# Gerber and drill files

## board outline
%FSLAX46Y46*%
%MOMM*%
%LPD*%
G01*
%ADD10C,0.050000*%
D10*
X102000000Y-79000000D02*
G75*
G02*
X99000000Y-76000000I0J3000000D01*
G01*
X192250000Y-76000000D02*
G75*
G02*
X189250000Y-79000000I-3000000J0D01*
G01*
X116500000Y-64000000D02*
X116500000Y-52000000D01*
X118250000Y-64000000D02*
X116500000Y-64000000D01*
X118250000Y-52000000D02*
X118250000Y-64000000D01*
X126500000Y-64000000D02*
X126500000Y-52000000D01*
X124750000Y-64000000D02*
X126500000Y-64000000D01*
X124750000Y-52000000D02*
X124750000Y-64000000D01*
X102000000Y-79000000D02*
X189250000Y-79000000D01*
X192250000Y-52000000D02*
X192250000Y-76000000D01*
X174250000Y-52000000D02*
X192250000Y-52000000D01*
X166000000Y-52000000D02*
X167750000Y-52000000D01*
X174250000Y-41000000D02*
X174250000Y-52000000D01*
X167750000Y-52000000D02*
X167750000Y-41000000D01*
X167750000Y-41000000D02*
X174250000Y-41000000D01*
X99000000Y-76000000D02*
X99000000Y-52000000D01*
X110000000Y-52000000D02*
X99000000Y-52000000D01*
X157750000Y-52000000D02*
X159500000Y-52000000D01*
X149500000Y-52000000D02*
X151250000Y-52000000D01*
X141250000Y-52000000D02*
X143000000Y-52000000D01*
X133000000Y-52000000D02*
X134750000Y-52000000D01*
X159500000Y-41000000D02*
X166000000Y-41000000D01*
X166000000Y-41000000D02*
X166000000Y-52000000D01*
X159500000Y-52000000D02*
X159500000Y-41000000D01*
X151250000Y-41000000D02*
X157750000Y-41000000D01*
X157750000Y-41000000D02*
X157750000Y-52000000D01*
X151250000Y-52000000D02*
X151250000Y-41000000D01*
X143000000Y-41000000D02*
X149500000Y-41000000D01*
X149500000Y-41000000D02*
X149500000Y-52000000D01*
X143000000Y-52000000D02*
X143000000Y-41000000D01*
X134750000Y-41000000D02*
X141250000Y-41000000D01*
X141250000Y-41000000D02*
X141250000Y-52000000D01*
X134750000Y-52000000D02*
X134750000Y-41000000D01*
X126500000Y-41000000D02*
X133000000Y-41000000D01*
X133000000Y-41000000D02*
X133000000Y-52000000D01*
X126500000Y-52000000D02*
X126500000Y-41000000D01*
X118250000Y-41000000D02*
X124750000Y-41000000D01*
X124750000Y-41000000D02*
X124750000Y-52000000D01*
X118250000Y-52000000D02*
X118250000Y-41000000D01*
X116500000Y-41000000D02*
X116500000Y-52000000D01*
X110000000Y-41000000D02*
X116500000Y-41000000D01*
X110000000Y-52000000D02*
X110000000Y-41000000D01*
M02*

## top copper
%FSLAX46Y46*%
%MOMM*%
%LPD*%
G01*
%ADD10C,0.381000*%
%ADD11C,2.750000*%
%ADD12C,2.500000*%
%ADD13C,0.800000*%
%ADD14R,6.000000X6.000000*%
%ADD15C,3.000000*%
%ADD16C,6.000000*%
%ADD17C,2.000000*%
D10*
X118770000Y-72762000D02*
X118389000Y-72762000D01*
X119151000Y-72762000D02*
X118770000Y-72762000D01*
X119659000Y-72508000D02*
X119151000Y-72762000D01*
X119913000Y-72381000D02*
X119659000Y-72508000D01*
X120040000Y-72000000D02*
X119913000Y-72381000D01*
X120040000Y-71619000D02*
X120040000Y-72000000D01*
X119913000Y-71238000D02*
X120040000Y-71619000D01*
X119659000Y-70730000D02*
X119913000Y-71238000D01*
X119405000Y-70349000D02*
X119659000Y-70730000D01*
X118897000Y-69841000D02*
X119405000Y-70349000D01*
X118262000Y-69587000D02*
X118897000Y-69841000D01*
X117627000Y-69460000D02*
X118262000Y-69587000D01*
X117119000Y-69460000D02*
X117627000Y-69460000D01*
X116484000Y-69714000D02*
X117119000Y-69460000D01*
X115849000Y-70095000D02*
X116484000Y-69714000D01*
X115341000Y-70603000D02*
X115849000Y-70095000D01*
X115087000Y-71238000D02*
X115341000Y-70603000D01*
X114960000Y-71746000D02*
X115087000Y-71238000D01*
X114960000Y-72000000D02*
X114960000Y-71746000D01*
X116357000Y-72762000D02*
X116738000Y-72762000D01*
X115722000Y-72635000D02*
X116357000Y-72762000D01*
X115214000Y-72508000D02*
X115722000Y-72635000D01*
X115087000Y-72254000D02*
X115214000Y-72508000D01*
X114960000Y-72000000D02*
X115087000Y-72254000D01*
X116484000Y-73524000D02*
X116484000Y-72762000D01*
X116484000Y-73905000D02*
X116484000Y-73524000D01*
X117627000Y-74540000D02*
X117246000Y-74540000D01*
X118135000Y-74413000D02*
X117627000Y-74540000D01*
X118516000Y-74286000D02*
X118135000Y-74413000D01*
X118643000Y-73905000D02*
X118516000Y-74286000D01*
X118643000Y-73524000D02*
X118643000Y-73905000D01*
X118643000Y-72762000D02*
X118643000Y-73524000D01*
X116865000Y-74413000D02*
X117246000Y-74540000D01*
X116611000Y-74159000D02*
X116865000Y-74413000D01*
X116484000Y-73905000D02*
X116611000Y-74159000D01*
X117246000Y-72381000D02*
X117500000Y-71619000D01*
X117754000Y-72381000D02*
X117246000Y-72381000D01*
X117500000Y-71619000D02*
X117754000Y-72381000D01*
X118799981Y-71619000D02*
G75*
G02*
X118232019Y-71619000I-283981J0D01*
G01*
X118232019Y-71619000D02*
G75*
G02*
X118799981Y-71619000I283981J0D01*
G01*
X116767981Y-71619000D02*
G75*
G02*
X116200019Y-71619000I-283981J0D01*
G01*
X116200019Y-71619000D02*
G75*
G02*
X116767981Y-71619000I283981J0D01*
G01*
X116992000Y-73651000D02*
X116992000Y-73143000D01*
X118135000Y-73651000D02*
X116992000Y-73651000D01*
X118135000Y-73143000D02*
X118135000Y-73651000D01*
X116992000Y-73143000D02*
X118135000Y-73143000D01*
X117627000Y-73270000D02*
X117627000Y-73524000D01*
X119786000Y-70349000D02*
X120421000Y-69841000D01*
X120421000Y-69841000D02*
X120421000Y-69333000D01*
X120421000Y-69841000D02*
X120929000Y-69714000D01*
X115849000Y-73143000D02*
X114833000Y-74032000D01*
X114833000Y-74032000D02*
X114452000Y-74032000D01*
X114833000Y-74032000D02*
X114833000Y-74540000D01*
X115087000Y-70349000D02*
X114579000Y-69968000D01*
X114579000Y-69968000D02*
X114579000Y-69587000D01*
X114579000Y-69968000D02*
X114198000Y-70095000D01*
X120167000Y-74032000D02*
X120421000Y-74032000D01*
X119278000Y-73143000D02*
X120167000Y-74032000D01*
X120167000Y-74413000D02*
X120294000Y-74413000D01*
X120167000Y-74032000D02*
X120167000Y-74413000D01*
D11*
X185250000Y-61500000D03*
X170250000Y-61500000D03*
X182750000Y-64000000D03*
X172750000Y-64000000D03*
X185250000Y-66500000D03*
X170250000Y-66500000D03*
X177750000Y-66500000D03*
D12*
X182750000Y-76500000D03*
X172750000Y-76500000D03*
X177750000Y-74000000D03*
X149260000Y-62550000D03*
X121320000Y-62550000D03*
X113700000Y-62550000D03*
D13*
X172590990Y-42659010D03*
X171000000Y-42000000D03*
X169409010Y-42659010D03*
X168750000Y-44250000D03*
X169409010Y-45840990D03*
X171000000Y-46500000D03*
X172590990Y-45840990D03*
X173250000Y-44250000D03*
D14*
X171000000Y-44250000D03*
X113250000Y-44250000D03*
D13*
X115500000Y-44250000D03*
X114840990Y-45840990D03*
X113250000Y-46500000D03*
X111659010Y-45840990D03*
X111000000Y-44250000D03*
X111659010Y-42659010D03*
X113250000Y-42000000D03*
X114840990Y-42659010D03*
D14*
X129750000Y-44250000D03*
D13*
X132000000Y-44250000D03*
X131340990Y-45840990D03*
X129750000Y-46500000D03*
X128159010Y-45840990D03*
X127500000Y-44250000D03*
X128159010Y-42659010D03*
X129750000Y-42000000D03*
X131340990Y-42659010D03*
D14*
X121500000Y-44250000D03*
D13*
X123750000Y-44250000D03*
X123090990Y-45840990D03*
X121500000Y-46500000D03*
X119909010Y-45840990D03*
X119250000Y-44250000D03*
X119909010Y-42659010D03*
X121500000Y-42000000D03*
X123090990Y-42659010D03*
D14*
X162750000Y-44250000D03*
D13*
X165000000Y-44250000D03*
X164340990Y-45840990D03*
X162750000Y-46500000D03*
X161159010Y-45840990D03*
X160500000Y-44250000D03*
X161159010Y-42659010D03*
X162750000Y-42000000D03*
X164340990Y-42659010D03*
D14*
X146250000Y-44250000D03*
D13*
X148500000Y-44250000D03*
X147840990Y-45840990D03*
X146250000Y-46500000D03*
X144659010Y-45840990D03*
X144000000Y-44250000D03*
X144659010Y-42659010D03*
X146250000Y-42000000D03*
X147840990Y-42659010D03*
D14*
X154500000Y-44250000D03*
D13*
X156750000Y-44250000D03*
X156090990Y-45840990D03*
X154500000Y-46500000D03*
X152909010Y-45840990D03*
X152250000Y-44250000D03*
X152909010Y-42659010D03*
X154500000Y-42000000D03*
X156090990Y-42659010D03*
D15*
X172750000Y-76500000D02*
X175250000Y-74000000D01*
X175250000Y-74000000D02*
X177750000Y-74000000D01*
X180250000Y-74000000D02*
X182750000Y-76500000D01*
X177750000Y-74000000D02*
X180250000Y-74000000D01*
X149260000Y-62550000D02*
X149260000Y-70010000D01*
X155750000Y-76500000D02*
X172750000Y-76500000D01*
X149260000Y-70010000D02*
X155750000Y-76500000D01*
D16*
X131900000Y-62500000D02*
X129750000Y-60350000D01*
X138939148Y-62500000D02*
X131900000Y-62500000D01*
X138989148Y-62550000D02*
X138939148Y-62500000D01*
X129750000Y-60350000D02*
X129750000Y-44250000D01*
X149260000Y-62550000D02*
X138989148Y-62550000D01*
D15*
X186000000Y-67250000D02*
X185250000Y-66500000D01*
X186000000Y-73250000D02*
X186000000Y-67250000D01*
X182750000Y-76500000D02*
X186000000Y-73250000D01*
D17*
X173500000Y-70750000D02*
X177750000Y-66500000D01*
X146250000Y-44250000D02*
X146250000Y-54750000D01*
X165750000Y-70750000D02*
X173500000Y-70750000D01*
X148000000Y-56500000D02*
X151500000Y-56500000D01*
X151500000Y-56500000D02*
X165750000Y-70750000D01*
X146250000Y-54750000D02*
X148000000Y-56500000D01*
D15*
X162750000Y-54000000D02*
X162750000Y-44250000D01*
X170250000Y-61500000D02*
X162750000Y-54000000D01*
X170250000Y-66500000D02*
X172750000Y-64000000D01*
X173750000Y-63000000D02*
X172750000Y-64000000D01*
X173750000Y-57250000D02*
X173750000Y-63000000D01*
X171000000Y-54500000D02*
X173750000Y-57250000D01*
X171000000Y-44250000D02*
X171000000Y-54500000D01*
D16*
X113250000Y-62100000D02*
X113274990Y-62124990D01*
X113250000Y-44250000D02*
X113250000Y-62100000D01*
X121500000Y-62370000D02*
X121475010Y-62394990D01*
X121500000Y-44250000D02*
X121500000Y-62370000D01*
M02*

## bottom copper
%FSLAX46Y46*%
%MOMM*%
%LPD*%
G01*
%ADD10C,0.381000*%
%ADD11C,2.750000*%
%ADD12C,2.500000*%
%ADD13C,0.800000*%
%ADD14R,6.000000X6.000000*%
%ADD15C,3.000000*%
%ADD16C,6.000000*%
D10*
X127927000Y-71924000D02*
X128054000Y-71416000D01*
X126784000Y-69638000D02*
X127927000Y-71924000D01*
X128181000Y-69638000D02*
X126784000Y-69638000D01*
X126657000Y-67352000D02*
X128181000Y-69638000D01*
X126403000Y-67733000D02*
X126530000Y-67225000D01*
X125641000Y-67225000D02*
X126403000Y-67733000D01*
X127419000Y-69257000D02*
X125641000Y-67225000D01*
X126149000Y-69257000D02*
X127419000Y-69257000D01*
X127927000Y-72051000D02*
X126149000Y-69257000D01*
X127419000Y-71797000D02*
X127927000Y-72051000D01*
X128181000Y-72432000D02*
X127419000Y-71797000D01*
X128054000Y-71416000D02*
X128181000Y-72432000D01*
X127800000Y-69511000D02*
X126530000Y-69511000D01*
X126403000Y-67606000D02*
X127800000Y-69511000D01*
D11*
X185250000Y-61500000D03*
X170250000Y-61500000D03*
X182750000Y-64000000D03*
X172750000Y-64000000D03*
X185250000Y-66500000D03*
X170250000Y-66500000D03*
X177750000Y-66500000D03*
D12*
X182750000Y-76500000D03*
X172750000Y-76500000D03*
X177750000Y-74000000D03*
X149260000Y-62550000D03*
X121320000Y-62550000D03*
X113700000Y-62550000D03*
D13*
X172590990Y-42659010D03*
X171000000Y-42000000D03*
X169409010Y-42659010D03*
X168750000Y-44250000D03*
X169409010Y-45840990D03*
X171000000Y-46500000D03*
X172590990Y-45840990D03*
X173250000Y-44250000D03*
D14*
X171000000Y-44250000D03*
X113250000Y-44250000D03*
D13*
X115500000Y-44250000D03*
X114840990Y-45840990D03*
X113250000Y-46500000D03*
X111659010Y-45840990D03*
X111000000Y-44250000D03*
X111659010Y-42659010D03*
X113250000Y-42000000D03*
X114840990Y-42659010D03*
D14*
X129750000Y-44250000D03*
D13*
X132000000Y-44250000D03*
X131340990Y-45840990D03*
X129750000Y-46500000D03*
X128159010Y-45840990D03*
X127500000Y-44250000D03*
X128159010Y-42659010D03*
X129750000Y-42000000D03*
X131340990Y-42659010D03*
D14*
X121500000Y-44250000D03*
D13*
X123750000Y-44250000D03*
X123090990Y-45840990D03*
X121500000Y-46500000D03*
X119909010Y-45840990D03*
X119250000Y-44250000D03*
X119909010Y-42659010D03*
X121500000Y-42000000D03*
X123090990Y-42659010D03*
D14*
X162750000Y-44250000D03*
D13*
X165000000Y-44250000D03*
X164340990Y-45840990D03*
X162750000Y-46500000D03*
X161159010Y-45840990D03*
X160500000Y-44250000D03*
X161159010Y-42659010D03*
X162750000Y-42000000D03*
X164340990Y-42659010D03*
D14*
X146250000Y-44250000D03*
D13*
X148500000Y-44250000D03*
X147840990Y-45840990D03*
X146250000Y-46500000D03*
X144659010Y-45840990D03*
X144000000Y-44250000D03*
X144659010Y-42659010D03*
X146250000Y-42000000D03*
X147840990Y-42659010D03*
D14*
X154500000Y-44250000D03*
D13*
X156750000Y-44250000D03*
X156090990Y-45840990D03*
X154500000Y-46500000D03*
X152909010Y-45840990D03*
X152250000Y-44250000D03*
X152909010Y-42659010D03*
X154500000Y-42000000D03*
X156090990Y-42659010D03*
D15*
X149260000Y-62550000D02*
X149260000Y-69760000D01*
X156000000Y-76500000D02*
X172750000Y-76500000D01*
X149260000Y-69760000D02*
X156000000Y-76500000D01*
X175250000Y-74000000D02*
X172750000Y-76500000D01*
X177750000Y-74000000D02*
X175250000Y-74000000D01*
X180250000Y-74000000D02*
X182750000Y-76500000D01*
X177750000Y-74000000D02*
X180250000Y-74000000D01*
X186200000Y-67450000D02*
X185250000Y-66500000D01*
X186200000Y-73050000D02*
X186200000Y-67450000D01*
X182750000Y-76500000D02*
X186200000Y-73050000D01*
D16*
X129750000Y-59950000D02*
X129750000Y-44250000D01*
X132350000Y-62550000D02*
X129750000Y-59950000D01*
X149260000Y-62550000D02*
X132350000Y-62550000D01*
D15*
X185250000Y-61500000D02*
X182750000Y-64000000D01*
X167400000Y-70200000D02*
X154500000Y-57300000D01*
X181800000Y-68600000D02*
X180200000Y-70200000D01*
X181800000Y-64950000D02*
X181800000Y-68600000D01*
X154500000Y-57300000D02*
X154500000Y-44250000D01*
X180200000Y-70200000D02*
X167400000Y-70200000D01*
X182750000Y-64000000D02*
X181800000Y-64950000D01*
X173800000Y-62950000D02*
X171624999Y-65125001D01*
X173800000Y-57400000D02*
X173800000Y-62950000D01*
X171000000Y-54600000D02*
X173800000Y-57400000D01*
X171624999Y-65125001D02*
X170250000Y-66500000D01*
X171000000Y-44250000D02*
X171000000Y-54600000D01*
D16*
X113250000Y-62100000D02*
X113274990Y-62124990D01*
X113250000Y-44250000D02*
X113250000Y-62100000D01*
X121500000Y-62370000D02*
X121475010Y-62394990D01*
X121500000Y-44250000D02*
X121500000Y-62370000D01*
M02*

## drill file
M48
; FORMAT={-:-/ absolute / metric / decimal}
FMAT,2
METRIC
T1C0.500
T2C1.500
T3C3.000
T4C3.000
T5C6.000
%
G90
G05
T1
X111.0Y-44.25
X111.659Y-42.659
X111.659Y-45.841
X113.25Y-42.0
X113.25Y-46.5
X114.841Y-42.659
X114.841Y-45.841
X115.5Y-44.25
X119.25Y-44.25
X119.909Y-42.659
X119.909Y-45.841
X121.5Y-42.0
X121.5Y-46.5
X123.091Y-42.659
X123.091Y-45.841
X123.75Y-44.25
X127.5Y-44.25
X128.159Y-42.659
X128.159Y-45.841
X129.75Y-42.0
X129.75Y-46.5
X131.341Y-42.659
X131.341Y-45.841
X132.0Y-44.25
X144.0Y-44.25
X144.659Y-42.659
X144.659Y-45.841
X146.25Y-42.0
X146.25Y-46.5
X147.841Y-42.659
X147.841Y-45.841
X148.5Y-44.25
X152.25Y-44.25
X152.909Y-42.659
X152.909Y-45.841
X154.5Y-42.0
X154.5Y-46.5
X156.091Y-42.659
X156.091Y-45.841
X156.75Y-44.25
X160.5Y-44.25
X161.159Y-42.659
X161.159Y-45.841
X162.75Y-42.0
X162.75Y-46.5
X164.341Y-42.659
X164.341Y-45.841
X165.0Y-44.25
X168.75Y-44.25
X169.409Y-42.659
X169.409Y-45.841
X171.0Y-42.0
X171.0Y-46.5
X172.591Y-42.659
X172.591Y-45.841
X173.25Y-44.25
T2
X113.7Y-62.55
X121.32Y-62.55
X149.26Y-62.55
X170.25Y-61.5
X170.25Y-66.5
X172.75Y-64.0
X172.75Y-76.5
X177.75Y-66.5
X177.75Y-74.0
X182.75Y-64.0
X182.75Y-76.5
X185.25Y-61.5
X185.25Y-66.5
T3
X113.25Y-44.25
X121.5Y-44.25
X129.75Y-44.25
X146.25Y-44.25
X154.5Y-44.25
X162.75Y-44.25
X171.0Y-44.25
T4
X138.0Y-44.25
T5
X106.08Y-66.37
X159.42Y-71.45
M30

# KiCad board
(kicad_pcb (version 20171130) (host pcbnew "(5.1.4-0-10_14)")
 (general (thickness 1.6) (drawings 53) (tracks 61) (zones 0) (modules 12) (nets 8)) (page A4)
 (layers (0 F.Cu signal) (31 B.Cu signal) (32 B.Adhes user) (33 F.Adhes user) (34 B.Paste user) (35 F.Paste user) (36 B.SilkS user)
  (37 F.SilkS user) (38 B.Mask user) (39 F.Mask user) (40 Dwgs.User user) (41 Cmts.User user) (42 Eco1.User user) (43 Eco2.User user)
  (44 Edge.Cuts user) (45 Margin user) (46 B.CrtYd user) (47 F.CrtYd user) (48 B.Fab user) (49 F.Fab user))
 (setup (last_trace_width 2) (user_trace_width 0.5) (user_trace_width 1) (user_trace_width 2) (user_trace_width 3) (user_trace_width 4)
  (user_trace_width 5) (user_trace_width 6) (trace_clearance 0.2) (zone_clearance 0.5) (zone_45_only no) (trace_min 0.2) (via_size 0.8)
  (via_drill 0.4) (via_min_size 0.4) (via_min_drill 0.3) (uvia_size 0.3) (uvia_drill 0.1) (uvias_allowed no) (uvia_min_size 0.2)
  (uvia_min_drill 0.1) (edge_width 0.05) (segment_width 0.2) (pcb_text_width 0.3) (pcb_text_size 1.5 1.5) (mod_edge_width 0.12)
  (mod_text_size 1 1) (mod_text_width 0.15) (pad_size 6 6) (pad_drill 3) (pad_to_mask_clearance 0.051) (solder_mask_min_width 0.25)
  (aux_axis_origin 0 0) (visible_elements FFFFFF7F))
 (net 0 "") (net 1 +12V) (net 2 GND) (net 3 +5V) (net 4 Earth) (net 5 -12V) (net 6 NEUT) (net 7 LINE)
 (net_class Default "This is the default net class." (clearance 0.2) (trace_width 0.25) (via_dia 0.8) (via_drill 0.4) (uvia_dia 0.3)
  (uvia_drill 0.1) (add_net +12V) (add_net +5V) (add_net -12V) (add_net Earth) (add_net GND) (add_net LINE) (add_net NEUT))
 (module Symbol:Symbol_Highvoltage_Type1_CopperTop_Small (layer B.Cu) (at 127.8 70.4 180)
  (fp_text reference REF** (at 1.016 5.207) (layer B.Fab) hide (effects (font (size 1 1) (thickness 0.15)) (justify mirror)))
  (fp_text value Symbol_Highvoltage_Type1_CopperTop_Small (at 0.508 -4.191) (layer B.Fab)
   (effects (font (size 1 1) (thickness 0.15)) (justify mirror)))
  (fp_line (start -0.127 -1.524) (end -0.254 -1.016) (layer B.Cu) (width 0.381))
  (fp_line (start 1.016 0.762) (end -0.127 -1.524) (layer B.Cu) (width 0.381))
  (fp_line (start -0.381 0.762) (end 1.016 0.762) (layer B.Cu) (width 0.381))
  (fp_line (start 1.143 3.048) (end -0.381 0.762) (layer B.Cu) (width 0.381))
  (fp_line (start 1.397 2.667) (end 1.27 3.175) (layer B.Cu) (width 0.381))
  (fp_line (start 2.159 3.175) (end 1.397 2.667) (layer B.Cu) (width 0.381))
  (fp_line (start 0.381 1.143) (end 2.159 3.175) (layer B.Cu) (width 0.381))
  (fp_line (start 1.651 1.143) (end 0.381 1.143) (layer B.Cu) (width 0.381))
  (fp_line (start -0.127 -1.651) (end 1.651 1.143) (layer B.Cu) (width 0.381))
  (fp_line (start 0.381 -1.397) (end -0.127 -1.651) (layer B.Cu) (width 0.381))
  (fp_line (start -0.381 -2.032) (end 0.381 -1.397) (layer B.Cu) (width 0.381))
  (fp_line (start -0.254 -1.016) (end -0.381 -2.032) (layer B.Cu) (width 0.381))
  (fp_line (start 0 0.889) (end 1.27 0.889) (layer B.Cu) (width 0.381))
  (fp_line (start 1.397 2.794) (end 0 0.889) (layer B.Cu) (width 0.381)))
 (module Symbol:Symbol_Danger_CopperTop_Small (layer F.Cu) (at 117.5 72)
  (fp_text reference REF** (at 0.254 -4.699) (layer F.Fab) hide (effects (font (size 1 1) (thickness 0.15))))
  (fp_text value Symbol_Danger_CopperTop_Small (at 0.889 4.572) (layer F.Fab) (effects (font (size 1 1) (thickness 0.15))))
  (fp_line (start 1.27 0.762) (end 0.889 0.762) (layer F.Cu) (width 0.381))
  (fp_line (start 1.651 0.762) (end 1.27 0.762) (layer F.Cu) (width 0.381))
  (fp_line (start 2.159 0.508) (end 1.651 0.762) (layer F.Cu) (width 0.381))
  (fp_line (start 2.413 0.381) (end 2.159 0.508) (layer F.Cu) (width 0.381))
  (fp_line (start 2.54 0) (end 2.413 0.381) (layer F.Cu) (width 0.381))
  (fp_line (start 2.54 -0.381) (end 2.54 0) (layer F.Cu) (width 0.381))
  (fp_line (start 2.413 -0.762) (end 2.54 -0.381) (layer F.Cu) (width 0.381))
  (fp_line (start 2.159 -1.27) (end 2.413 -0.762) (layer F.Cu) (width 0.381))
  (fp_line (start 1.905 -1.651) (end 2.159 -1.27) (layer F.Cu) (width 0.381))
  (fp_line (start 1.397 -2.159) (end 1.905 -1.651) (layer F.Cu) (width 0.381))
  (fp_line (start 0.762 -2.413) (end 1.397 -2.159) (layer F.Cu) (width 0.381))
  (fp_line (start 0.127 -2.54) (end 0.762 -2.413) (layer F.Cu) (width 0.381))
  (fp_line (start -0.381 -2.54) (end 0.127 -2.54) (layer F.Cu) (width 0.381))
  (fp_line (start -1.016 -2.286) (end -0.381 -2.54) (layer F.Cu) (width 0.381))
  (fp_line (start -1.651 -1.905) (end -1.016 -2.286) (layer F.Cu) (width 0.381))
  (fp_line (start -2.159 -1.397) (end -1.651 -1.905) (layer F.Cu) (width 0.381))
  (fp_line (start -2.413 -0.762) (end -2.159 -1.397) (layer F.Cu) (width 0.381))
  (fp_line (start -2.54 -0.254) (end -2.413 -0.762) (layer F.Cu) (width 0.381))
  (fp_line (start -2.54 0) (end -2.54 -0.254) (layer F.Cu) (width 0.381))
  (fp_line (start -1.143 0.762) (end -0.762 0.762) (layer F.Cu) (width 0.381))
  (fp_line (start -1.778 0.635) (end -1.143 0.762) (layer F.Cu) (width 0.381))
  (fp_line (start -2.286 0.508) (end -1.778 0.635) (layer F.Cu) (width 0.381))
  (fp_line (start -2.413 0.254) (end -2.286 0.508) (layer F.Cu) (width 0.381))
  (fp_line (start -2.54 0) (end -2.413 0.254) (layer F.Cu) (width 0.381))
  (fp_line (start -1.016 1.524) (end -1.016 0.762) (layer F.Cu) (width 0.381))
  (fp_line (start -1.016 1.905) (end -1.016 1.524) (layer F.Cu) (width 0.381))
  (fp_line (start 0.127 2.54) (end -0.254 2.54) (layer F.Cu) (width 0.381))
  (fp_line (start 0.635 2.413) (end 0.127 2.54) (layer F.Cu) (width 0.381))
  (fp_line (start 1.016 2.286) (end 0.635 2.413) (layer F.Cu) (width 0.381))
  (fp_line (start 1.143 1.905) (end 1.016 2.286) (layer F.Cu) (width 0.381))
  (fp_line (start 1.143 1.524) (end 1.143 1.905) (layer F.Cu) (width 0.381))
  (fp_line (start 1.143 0.762) (end 1.143 1.524) (layer F.Cu) (width 0.381))
  (fp_line (start -0.635 2.413) (end -0.254 2.54) (layer F.Cu) (width 0.381))
  (fp_line (start -0.889 2.159) (end -0.635 2.413) (layer F.Cu) (width 0.381))
  (fp_line (start -1.016 1.905) (end -0.889 2.159) (layer F.Cu) (width 0.381))
  (fp_line (start -0.254 0.381) (end 0 -0.381) (layer F.Cu) (width 0.381))
  (fp_line (start 0.254 0.381) (end -0.254 0.381) (layer F.Cu) (width 0.381))
  (fp_line (start 0 -0.381) (end 0.254 0.381) (layer F.Cu) (width 0.381))
  (fp_circle (center 1.016 -0.381) (end 1.27 -0.254) (layer F.Cu) (width 0.381))
  (fp_circle (center -1.016 -0.381) (end -1.27 -0.254) (layer F.Cu) (width 0.381))
  (fp_line (start -0.508 1.651) (end -0.508 1.143) (layer F.Cu) (width 0.381))
  (fp_line (start 0.635 1.651) (end -0.508 1.651) (layer F.Cu) (width 0.381))
  (fp_line (start 0.635 1.143) (end 0.635 1.651) (layer F.Cu) (width 0.381))
  (fp_line (start -0.508 1.143) (end 0.635 1.143) (layer F.Cu) (width 0.381))
  (fp_line (start 0.127 1.27) (end 0.127 1.524) (layer F.Cu) (width 0.381))
  (fp_line (start 2.286 -1.651) (end 2.921 -2.159) (layer F.Cu) (width 0.381))
  (fp_line (start 2.921 -2.159) (end 2.921 -2.667) (layer F.Cu) (width 0.381))
  (fp_line (start 2.921 -2.159) (end 3.429 -2.286) (layer F.Cu) (width 0.381))
  (fp_line (start -1.651 1.143) (end -2.667 2.032) (layer F.Cu) (width 0.381))
  (fp_line (start -2.667 2.032) (end -3.048 2.032) (layer F.Cu) (width 0.381))
  (fp_line (start -2.667 2.032) (end -2.667 2.54) (layer F.Cu) (width 0.381))
  (fp_line (start -2.413 -1.651) (end -2.921 -2.032) (layer F.Cu) (width 0.381))
  (fp_line (start -2.921 -2.032) (end -2.921 -2.413) (layer F.Cu) (width 0.381))
  (fp_line (start -2.921 -2.032) (end -3.302 -1.905) (layer F.Cu) (width 0.381))
  (fp_line (start 2.667 2.032) (end 2.921 2.032) (layer F.Cu) (width 0.381))
  (fp_line (start 1.778 1.143) (end 2.667 2.032) (layer F.Cu) (width 0.381))
  (fp_line (start 2.667 2.413) (end 2.794 2.413) (layer F.Cu) (width 0.381))
  (fp_line (start 2.667 2.032) (end 2.667 2.413) (layer F.Cu) (width 0.381)))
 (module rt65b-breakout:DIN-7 (layer F.Cu) (at 177.75 74)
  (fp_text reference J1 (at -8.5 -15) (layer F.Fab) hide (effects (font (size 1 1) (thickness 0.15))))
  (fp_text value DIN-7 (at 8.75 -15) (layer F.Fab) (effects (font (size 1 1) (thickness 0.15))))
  (pad 6 thru_hole circle (at 7.5 -12.5) (size 2.75 2.75) (drill 1.5) (layers *.Cu *.Mask) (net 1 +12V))
  (pad 7 thru_hole circle (at -7.5 -12.5) (size 2.75 2.75) (drill 1.5) (layers *.Cu *.Mask) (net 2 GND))
  (pad 4 thru_hole circle (at 5 -10 90) (size 2.75 2.75) (drill 1.5) (layers *.Cu *.Mask) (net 1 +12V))
  (pad 5 thru_hole circle (at -5 -10) (size 2.75 2.75) (drill 1.5) (layers *.Cu *.Mask) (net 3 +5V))
  (pad 1 thru_hole circle (at 7.5 -7.5) (size 2.75 2.75) (drill 1.5) (layers *.Cu *.Mask) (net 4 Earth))
  (pad 3 thru_hole circle (at -7.5 -7.5) (size 2.75 2.75) (drill 1.5) (layers *.Cu *.Mask) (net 3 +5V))
  (pad 2 thru_hole circle (at 0 -7.5) (size 2.75 2.75) (drill 1.5) (layers *.Cu *.Mask) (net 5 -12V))
  (pad 10 thru_hole circle (at 5 2.5) (size 2.5 2.5) (drill 1.5) (layers *.Cu *.Mask) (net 4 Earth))
  (pad 8 thru_hole circle (at -5 2.5) (size 2.5 2.5) (drill 1.5) (layers *.Cu *.Mask) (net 4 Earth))
  (pad 9 thru_hole circle (at 0 0) (size 2.5 2.5) (drill 1.5) (layers *.Cu *.Mask) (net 4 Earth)))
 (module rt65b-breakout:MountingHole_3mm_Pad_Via (layer F.Cu) (at 138 44.25)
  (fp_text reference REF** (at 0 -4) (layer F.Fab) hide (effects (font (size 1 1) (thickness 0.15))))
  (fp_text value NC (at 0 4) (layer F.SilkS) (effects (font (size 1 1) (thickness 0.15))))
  (pad "" np_thru_hole circle (at 0 0) (size 3 3) (drill 3) (layers *.Cu *.Mask)))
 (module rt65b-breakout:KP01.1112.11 (layer F.Cu) (at 132.75 79)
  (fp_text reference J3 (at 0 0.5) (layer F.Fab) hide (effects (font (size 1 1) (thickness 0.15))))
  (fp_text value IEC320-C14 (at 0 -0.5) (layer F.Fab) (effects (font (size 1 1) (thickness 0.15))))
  (pad 3 thru_hole circle (at 16.51 -16.45) (size 2.5 2.5) (drill 1.5) (layers *.Cu *.Mask) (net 4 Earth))
  (pad "" np_thru_hole circle (at -26.67 -12.63) (size 6 6) (drill 6) (layers *.Cu *.Mask))
  (pad "" np_thru_hole circle (at 26.67 -7.55) (size 6 6) (drill 6) (layers *.Cu *.Mask))
  (pad 2 thru_hole circle (at -11.43 -16.45) (size 2.5 2.5) (drill 1.5) (layers *.Cu *.Mask) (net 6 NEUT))
  (pad 1 thru_hole circle (at -19.05 -16.45) (size 2.5 2.5) (drill 1.5) (layers *.Cu *.Mask) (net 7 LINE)))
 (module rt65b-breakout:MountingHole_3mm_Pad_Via (layer F.Cu) (at 171 44.25)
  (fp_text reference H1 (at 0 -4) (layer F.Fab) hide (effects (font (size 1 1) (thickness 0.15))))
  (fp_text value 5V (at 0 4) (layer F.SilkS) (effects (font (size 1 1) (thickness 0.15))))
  (pad 1 thru_hole circle (at 1.59099 -1.59099) (size 0.8 0.8) (drill 0.5) (layers *.Cu *.Mask) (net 3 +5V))
  (pad 1 thru_hole circle (at 0 -2.25) (size 0.8 0.8) (drill 0.5) (layers *.Cu *.Mask) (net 3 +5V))
  (pad 1 thru_hole circle (at -1.59099 -1.59099) (size 0.8 0.8) (drill 0.5) (layers *.Cu *.Mask) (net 3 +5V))
  (pad 1 thru_hole circle (at -2.25 0) (size 0.8 0.8) (drill 0.5) (layers *.Cu *.Mask) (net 3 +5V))
  (pad 1 thru_hole circle (at -1.59099 1.59099) (size 0.8 0.8) (drill 0.5) (layers *.Cu *.Mask) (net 3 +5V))
  (pad 1 thru_hole circle (at 0 2.25) (size 0.8 0.8) (drill 0.5) (layers *.Cu *.Mask) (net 3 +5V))
  (pad 1 thru_hole circle (at 1.59099 1.59099) (size 0.8 0.8) (drill 0.5) (layers *.Cu *.Mask) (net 3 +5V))
  (pad 1 thru_hole circle (at 2.25 0) (size 0.8 0.8) (drill 0.5) (layers *.Cu *.Mask) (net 3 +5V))
  (pad 1 thru_hole rect (at 0 0) (size 6 6) (drill 3) (layers *.Cu *.Mask) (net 3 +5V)))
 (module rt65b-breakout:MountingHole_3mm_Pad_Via (layer F.Cu) (at 113.25 44.25)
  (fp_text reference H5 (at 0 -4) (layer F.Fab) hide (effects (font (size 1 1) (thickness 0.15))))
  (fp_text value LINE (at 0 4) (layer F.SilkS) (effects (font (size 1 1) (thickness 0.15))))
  (pad 1 thru_hole rect (at 0 0) (size 6 6) (drill 3) (layers *.Cu *.Mask) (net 7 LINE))
  (pad 1 thru_hole circle (at 2.25 0) (size 0.8 0.8) (drill 0.5) (layers *.Cu *.Mask) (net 7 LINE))
  (pad 1 thru_hole circle (at 1.59099 1.59099) (size 0.8 0.8) (drill 0.5) (layers *.Cu *.Mask) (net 7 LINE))
  (pad 1 thru_hole circle (at 0 2.25) (size 0.8 0.8) (drill 0.5) (layers *.Cu *.Mask) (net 7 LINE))
  (pad 1 thru_hole circle (at -1.59099 1.59099) (size 0.8 0.8) (drill 0.5) (layers *.Cu *.Mask) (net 7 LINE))
  (pad 1 thru_hole circle (at -2.25 0) (size 0.8 0.8) (drill 0.5) (layers *.Cu *.Mask) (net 7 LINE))
  (pad 1 thru_hole circle (at -1.59099 -1.59099) (size 0.8 0.8) (drill 0.5) (layers *.Cu *.Mask) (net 7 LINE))
  (pad 1 thru_hole circle (at 0 -2.25) (size 0.8 0.8) (drill 0.5) (layers *.Cu *.Mask) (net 7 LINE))
  (pad 1 thru_hole circle (at 1.59099 -1.59099) (size 0.8 0.8) (drill 0.5) (layers *.Cu *.Mask) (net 7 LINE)))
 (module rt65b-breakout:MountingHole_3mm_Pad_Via (layer F.Cu) (at 129.75 44.25)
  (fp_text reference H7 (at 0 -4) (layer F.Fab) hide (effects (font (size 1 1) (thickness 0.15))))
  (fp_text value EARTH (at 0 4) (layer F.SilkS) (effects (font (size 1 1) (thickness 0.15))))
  (pad 1 thru_hole rect (at 0 0) (size 6 6) (drill 3) (layers *.Cu *.Mask) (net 4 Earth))
  (pad 1 thru_hole circle (at 2.25 0) (size 0.8 0.8) (drill 0.5) (layers *.Cu *.Mask) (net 4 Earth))
  (pad 1 thru_hole circle (at 1.59099 1.59099) (size 0.8 0.8) (drill 0.5) (layers *.Cu *.Mask) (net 4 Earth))
  (pad 1 thru_hole circle (at 0 2.25) (size 0.8 0.8) (drill 0.5) (layers *.Cu *.Mask) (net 4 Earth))
  (pad 1 thru_hole circle (at -1.59099 1.59099) (size 0.8 0.8) (drill 0.5) (layers *.Cu *.Mask) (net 4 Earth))
  (pad 1 thru_hole circle (at -2.25 0) (size 0.8 0.8) (drill 0.5) (layers *.Cu *.Mask) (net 4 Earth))
  (pad 1 thru_hole circle (at -1.59099 -1.59099) (size 0.8 0.8) (drill 0.5) (layers *.Cu *.Mask) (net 4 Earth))
  (pad 1 thru_hole circle (at 0 -2.25) (size 0.8 0.8) (drill 0.5) (layers *.Cu *.Mask) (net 4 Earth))
  (pad 1 thru_hole circle (at 1.59099 -1.59099) (size 0.8 0.8) (drill 0.5) (layers *.Cu *.Mask) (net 4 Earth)))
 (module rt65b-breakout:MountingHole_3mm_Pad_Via (layer F.Cu) (at 121.5 44.25)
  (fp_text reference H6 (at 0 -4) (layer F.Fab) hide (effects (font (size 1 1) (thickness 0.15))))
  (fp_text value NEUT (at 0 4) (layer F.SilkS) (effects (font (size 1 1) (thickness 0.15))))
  (pad 1 thru_hole rect (at 0 0) (size 6 6) (drill 3) (layers *.Cu *.Mask) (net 6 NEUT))
  (pad 1 thru_hole circle (at 2.25 0) (size 0.8 0.8) (drill 0.5) (layers *.Cu *.Mask) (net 6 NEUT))
  (pad 1 thru_hole circle (at 1.59099 1.59099) (size 0.8 0.8) (drill 0.5) (layers *.Cu *.Mask) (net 6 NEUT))
  (pad 1 thru_hole circle (at 0 2.25) (size 0.8 0.8) (drill 0.5) (layers *.Cu *.Mask) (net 6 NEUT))
  (pad 1 thru_hole circle (at -1.59099 1.59099) (size 0.8 0.8) (drill 0.5) (layers *.Cu *.Mask) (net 6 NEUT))
  (pad 1 thru_hole circle (at -2.25 0) (size 0.8 0.8) (drill 0.5) (layers *.Cu *.Mask) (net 6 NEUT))
  (pad 1 thru_hole circle (at -1.59099 -1.59099) (size 0.8 0.8) (drill 0.5) (layers *.Cu *.Mask) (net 6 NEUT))
  (pad 1 thru_hole circle (at 0 -2.25) (size 0.8 0.8) (drill 0.5) (layers *.Cu *.Mask) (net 6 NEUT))
  (pad 1 thru_hole circle (at 1.59099 -1.59099) (size 0.8 0.8) (drill 0.5) (layers *.Cu *.Mask) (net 6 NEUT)))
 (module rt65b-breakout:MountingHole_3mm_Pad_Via (layer F.Cu) (at 162.75 44.25)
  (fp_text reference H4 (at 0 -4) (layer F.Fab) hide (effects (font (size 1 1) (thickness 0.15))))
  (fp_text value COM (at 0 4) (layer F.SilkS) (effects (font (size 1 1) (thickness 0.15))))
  (pad 1 thru_hole rect (at 0 0) (size 6 6) (drill 3) (layers *.Cu *.Mask) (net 2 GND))
  (pad 1 thru_hole circle (at 2.25 0) (size 0.8 0.8) (drill 0.5) (layers *.Cu *.Mask) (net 2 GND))
  (pad 1 thru_hole circle (at 1.59099 1.59099) (size 0.8 0.8) (drill 0.5) (layers *.Cu *.Mask) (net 2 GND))
  (pad 1 thru_hole circle (at 0 2.25) (size 0.8 0.8) (drill 0.5) (layers *.Cu *.Mask) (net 2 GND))
  (pad 1 thru_hole circle (at -1.59099 1.59099) (size 0.8 0.8) (drill 0.5) (layers *.Cu *.Mask) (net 2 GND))
  (pad 1 thru_hole circle (at -2.25 0) (size 0.8 0.8) (drill 0.5) (layers *.Cu *.Mask) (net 2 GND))
  (pad 1 thru_hole circle (at -1.59099 -1.59099) (size 0.8 0.8) (drill 0.5) (layers *.Cu *.Mask) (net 2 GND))
  (pad 1 thru_hole circle (at 0 -2.25) (size 0.8 0.8) (drill 0.5) (layers *.Cu *.Mask) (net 2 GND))
  (pad 1 thru_hole circle (at 1.59099 -1.59099) (size 0.8 0.8) (drill 0.5) (layers *.Cu *.Mask) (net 2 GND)))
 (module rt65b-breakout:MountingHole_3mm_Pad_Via (layer F.Cu) (at 146.25 44.25)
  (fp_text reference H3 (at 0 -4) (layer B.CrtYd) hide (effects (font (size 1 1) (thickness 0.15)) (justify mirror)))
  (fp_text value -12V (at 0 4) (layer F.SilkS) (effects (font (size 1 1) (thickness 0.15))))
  (pad 1 thru_hole rect (at 0 0) (size 6 6) (drill 3) (layers *.Cu *.Mask) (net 5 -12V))
  (pad 1 thru_hole circle (at 2.25 0) (size 0.8 0.8) (drill 0.5) (layers *.Cu *.Mask) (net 5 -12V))
  (pad 1 thru_hole circle (at 1.59099 1.59099) (size 0.8 0.8) (drill 0.5) (layers *.Cu *.Mask) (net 5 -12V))
  (pad 1 thru_hole circle (at 0 2.25) (size 0.8 0.8) (drill 0.5) (layers *.Cu *.Mask) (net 5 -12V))
  (pad 1 thru_hole circle (at -1.59099 1.59099) (size 0.8 0.8) (drill 0.5) (layers *.Cu *.Mask) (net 5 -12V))
  (pad 1 thru_hole circle (at -2.25 0) (size 0.8 0.8) (drill 0.5) (layers *.Cu *.Mask) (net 5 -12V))
  (pad 1 thru_hole circle (at -1.59099 -1.59099) (size 0.8 0.8) (drill 0.5) (layers *.Cu *.Mask) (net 5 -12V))
  (pad 1 thru_hole circle (at 0 -2.25) (size 0.8 0.8) (drill 0.5) (layers *.Cu *.Mask) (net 5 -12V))
  (pad 1 thru_hole circle (at 1.59099 -1.59099) (size 0.8 0.8) (drill 0.5) (layers *.Cu *.Mask) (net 5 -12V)))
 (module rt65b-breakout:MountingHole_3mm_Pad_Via (layer F.Cu) (at 154.5 44.25)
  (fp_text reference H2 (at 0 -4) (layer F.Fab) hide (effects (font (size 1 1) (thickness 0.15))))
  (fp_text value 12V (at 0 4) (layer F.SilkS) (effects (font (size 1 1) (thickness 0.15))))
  (pad 1 thru_hole rect (at 0 0) (size 6 6) (drill 3) (layers *.Cu *.Mask) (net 1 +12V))
  (pad 1 thru_hole circle (at 2.25 0) (size 0.8 0.8) (drill 0.5) (layers *.Cu *.Mask) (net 1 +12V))
  (pad 1 thru_hole circle (at 1.59099 1.59099) (size 0.8 0.8) (drill 0.5) (layers *.Cu *.Mask) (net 1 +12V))
  (pad 1 thru_hole circle (at 0 2.25) (size 0.8 0.8) (drill 0.5) (layers *.Cu *.Mask) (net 1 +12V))
  (pad 1 thru_hole circle (at -1.59099 1.59099) (size 0.8 0.8) (drill 0.5) (layers *.Cu *.Mask) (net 1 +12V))
  (pad 1 thru_hole circle (at -2.25 0) (size 0.8 0.8) (drill 0.5) (layers *.Cu *.Mask) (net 1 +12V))
  (pad 1 thru_hole circle (at -1.59099 -1.59099) (size 0.8 0.8) (drill 0.5) (layers *.Cu *.Mask) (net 1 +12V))
  (pad 1 thru_hole circle (at 0 -2.25) (size 0.8 0.8) (drill 0.5) (layers *.Cu *.Mask) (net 1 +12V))
  (pad 1 thru_hole circle (at 1.59099 -1.59099) (size 0.8 0.8) (drill 0.5) (layers *.Cu *.Mask) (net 1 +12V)))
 (gr_arc (start 102 76) (end 99 76) (angle -90) (layer Edge.Cuts) (width 0.05))
 (gr_arc (start 189.25 76) (end 189.25 79) (angle -90) (layer Edge.Cuts) (width 0.05))
 (gr_line (start 116.5 64) (end 116.5 52) (layer Edge.Cuts) (width 0.05))
 (gr_line (start 118.25 64) (end 116.5 64) (layer Edge.Cuts) (width 0.05))
 (gr_line (start 118.25 52) (end 118.25 64) (layer Edge.Cuts) (width 0.05))
 (gr_line (start 126.5 64) (end 126.5 52) (layer Edge.Cuts) (width 0.05))
 (gr_line (start 124.75 64) (end 126.5 64) (layer Edge.Cuts) (width 0.05))
 (gr_line (start 124.75 52) (end 124.75 64) (layer Edge.Cuts) (width 0.05))
 (gr_line (start 102 79) (end 189.25 79) (layer Edge.Cuts) (width 0.05))
 (gr_line (start 192.25 52) (end 192.25 76) (layer Edge.Cuts) (width 0.05))
 (gr_line (start 174.25 52) (end 192.25 52) (layer Edge.Cuts) (width 0.05))
 (gr_line (start 166 52) (end 167.75 52) (layer Edge.Cuts) (width 0.05))
 (gr_line (start 174.25 41) (end 174.25 52) (layer Edge.Cuts) (width 0.05))
 (gr_line (start 167.75 52) (end 167.75 41) (layer Edge.Cuts) (width 0.05))
 (gr_line (start 167.75 41) (end 174.25 41) (layer Edge.Cuts) (width 0.05))
 (gr_line (start 99 76) (end 99 52) (layer Edge.Cuts) (width 0.05))
 (gr_line (start 110 52) (end 99 52) (layer Edge.Cuts) (width 0.05))
 (gr_line (start 157.75 52) (end 159.5 52) (layer Edge.Cuts) (width 0.05))
 (gr_line (start 149.5 52) (end 151.25 52) (layer Edge.Cuts) (width 0.05))
 (gr_line (start 141.25 52) (end 143 52) (layer Edge.Cuts) (width 0.05))
 (gr_line (start 133 52) (end 134.75 52) (layer Edge.Cuts) (width 0.05))
 (gr_line (start 159.5 41) (end 166 41) (layer Edge.Cuts) (width 0.05))
 (gr_line (start 166 41) (end 166 52) (layer Edge.Cuts) (width 0.05))
 (gr_line (start 159.5 52) (end 159.5 41) (layer Edge.Cuts) (width 0.05))
 (gr_line (start 151.25 41) (end 157.75 41) (layer Edge.Cuts) (width 0.05))
 (gr_line (start 157.75 41) (end 157.75 52) (layer Edge.Cuts) (width 0.05))
 (gr_line (start 151.25 52) (end 151.25 41) (layer Edge.Cuts) (width 0.05))
 (gr_line (start 143 41) (end 149.5 41) (layer Edge.Cuts) (width 0.05))
 (gr_line (start 149.5 41) (end 149.5 52) (layer Edge.Cuts) (width 0.05))
 (gr_line (start 143 52) (end 143 41) (layer Edge.Cuts) (width 0.05))
 (gr_line (start 134.75 41) (end 141.25 41) (layer Edge.Cuts) (width 0.05))
 (gr_line (start 141.25 41) (end 141.25 52) (layer Edge.Cuts) (width 0.05))
 (gr_line (start 134.75 52) (end 134.75 41) (layer Edge.Cuts) (width 0.05))
 (gr_line (start 126.5 41) (end 133 41) (layer Edge.Cuts) (width 0.05))
 (gr_line (start 133 41) (end 133 52) (layer Edge.Cuts) (width 0.05))
 (gr_line (start 126.5 52) (end 126.5 41) (layer Edge.Cuts) (width 0.05))
 (gr_line (start 118.25 41) (end 124.75 41) (layer Edge.Cuts) (width 0.05))
 (gr_line (start 124.75 41) (end 124.75 52) (layer Edge.Cuts) (width 0.05))
 (gr_line (start 118.25 52) (end 118.25 41) (layer Edge.Cuts) (width 0.05))
 (gr_line (start 116.5 41) (end 116.5 52) (layer Edge.Cuts) (width 0.05))
 (gr_line (start 110 41) (end 116.5 41) (layer Edge.Cuts) (width 0.05))
 (gr_line (start 110 52) (end 110 41) (layer Edge.Cuts) (width 0.05))
 (segment (start 149.26 62.55) (end 149.26 69.76) (width 3) (layer B.Cu) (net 4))
 (segment (start 156 76.5) (end 172.75 76.5) (width 3) (layer B.Cu) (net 4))
 (segment (start 149.26 69.76) (end 156 76.5) (width 3) (layer B.Cu) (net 4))
 (segment (start 175.25 74) (end 172.75 76.5) (width 3) (layer B.Cu) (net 4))
 (segment (start 177.75 74) (end 175.25 74) (width 3) (layer B.Cu) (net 4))
 (segment (start 180.25 74) (end 182.75 76.5) (width 3) (layer B.Cu) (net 4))
 (segment (start 177.75 74) (end 180.25 74) (width 3) (layer B.Cu) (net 4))
 (segment (start 172.75 76.5) (end 175.25 74) (width 3) (layer F.Cu) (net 4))
 (segment (start 175.25 74) (end 177.75 74) (width 3) (layer F.Cu) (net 4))
 (segment (start 180.25 74) (end 182.75 76.5) (width 3) (layer F.Cu) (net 4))
 (segment (start 177.75 74) (end 180.25 74) (width 3) (layer F.Cu) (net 4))
 (segment (start 149.26 62.55) (end 149.26 70.01) (width 3) (layer F.Cu) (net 4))
 (segment (start 155.75 76.5) (end 172.75 76.5) (width 3) (layer F.Cu) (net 4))
 (segment (start 149.26 70.01) (end 155.75 76.5) (width 3) (layer F.Cu) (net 4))
 (segment (start 186.2 67.45) (end 185.25 66.5) (width 3) (layer B.Cu) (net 4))
 (segment (start 186.2 73.05) (end 186.2 67.45) (width 3) (layer B.Cu) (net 4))
 (segment (start 182.75 76.5) (end 186.2 73.05) (width 3) (layer B.Cu) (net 4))
 (segment (start 129.75 59.95) (end 129.75 44.25) (width 6) (layer B.Cu) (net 4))
 (segment (start 132.35 62.55) (end 129.75 59.95) (width 6) (layer B.Cu) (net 4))
 (segment (start 149.26 62.55) (end 132.35 62.55) (width 6) (layer B.Cu) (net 4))
 (segment (start 131.9 62.5) (end 129.75 60.35) (width 6) (layer F.Cu) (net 4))
 (segment (start 138.939148 62.5) (end 131.9 62.5) (width 6) (layer F.Cu) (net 4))
 (segment (start 138.989148 62.55) (end 138.939148 62.5) (width 6) (layer F.Cu) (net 4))
 (segment (start 129.75 60.35) (end 129.75 44.25) (width 6) (layer F.Cu) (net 4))
 (segment (start 149.26 62.55) (end 138.989148 62.55) (width 6) (layer F.Cu) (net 4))
 (segment (start 186 67.25) (end 185.25 66.5) (width 3) (layer F.Cu) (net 4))
 (segment (start 186 73.25) (end 186 67.25) (width 3) (layer F.Cu) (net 4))
 (segment (start 182.75 76.5) (end 186 73.25) (width 3) (layer F.Cu) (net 4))
 (segment (start 185.25 61.5) (end 182.75 64) (width 3) (layer B.Cu) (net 1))
 (segment (start 167.4 70.2) (end 154.5 57.3) (width 3) (layer B.Cu) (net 1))
 (segment (start 181.8 68.6) (end 180.2 70.2) (width 3) (layer B.Cu) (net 1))
 (segment (start 181.8 64.95) (end 181.8 68.6) (width 3) (layer B.Cu) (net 1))
 (segment (start 154.5 57.3) (end 154.5 44.25) (width 3) (layer B.Cu) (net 1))
 (segment (start 180.2 70.2) (end 167.4 70.2) (width 3) (layer B.Cu) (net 1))
 (segment (start 182.75 64) (end 181.8 64.95) (width 3) (layer B.Cu) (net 1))
 (segment (start 173.5 70.75) (end 177.75 66.5) (width 2) (layer F.Cu) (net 5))
 (segment (start 146.25 44.25) (end 146.25 54.75) (width 2) (layer F.Cu) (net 5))
 (segment (start 165.75 70.75) (end 173.5 70.75) (width 2) (layer F.Cu) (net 5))
 (segment (start 148 56.5) (end 151.5 56.5) (width 2) (layer F.Cu) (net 5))
 (segment (start 151.5 56.5) (end 165.75 70.75) (width 2) (layer F.Cu) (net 5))
 (segment (start 146.25 54.75) (end 148 56.5) (width 2) (layer F.Cu) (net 5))
 (segment (start 162.75 54) (end 162.75 44.25) (width 3) (layer F.Cu) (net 2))
 (segment (start 170.25 61.5) (end 162.75 54) (width 3) (layer F.Cu) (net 2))
 (segment (start 170.25 66.5) (end 172.75 64) (width 3) (layer F.Cu) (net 3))
 (segment (start 173.75 63) (end 172.75 64) (width 3) (layer F.Cu) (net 3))
 (segment (start 173.75 57.25) (end 173.75 63) (width 3) (layer F.Cu) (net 3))
 (segment (start 171 54.5) (end 173.75 57.25) (width 3) (layer F.Cu) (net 3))
 (segment (start 171 44.25) (end 171 54.5) (width 3) (layer F.Cu) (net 3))
 (segment (start 173.8 62.95) (end 171.624999 65.125001) (width 3) (layer B.Cu) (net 3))
 (segment (start 173.8 57.4) (end 173.8 62.95) (width 3) (layer B.Cu) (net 3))
 (segment (start 171 54.6) (end 173.8 57.4) (width 3) (layer B.Cu) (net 3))
 (segment (start 171.624999 65.125001) (end 170.25 66.5) (width 3) (layer B.Cu) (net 3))
 (segment (start 171 44.25) (end 171 54.6) (width 3) (layer B.Cu) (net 3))
 (segment (start 113.25 62.1) (end 113.27499 62.12499) (width 6) (layer F.Cu) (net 7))
 (segment (start 113.25 44.25) (end 113.25 62.1) (width 6) (layer F.Cu) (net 7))
 (segment (start 113.25 62.1) (end 113.27499 62.12499) (width 6) (layer B.Cu) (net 7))
 (segment (start 113.25 44.25) (end 113.25 62.1) (width 6) (layer B.Cu) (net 7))
 (segment (start 121.5 62.37) (end 121.47501 62.39499) (width 6) (layer F.Cu) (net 6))
 (segment (start 121.5 44.25) (end 121.5 62.37) (width 6) (layer F.Cu) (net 6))
 (segment (start 121.5 62.37) (end 121.47501 62.39499) (width 6) (layer B.Cu) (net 6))
 (segment (start 121.5 44.25) (end 121.5 62.37) (width 6) (layer B.Cu) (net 6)))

